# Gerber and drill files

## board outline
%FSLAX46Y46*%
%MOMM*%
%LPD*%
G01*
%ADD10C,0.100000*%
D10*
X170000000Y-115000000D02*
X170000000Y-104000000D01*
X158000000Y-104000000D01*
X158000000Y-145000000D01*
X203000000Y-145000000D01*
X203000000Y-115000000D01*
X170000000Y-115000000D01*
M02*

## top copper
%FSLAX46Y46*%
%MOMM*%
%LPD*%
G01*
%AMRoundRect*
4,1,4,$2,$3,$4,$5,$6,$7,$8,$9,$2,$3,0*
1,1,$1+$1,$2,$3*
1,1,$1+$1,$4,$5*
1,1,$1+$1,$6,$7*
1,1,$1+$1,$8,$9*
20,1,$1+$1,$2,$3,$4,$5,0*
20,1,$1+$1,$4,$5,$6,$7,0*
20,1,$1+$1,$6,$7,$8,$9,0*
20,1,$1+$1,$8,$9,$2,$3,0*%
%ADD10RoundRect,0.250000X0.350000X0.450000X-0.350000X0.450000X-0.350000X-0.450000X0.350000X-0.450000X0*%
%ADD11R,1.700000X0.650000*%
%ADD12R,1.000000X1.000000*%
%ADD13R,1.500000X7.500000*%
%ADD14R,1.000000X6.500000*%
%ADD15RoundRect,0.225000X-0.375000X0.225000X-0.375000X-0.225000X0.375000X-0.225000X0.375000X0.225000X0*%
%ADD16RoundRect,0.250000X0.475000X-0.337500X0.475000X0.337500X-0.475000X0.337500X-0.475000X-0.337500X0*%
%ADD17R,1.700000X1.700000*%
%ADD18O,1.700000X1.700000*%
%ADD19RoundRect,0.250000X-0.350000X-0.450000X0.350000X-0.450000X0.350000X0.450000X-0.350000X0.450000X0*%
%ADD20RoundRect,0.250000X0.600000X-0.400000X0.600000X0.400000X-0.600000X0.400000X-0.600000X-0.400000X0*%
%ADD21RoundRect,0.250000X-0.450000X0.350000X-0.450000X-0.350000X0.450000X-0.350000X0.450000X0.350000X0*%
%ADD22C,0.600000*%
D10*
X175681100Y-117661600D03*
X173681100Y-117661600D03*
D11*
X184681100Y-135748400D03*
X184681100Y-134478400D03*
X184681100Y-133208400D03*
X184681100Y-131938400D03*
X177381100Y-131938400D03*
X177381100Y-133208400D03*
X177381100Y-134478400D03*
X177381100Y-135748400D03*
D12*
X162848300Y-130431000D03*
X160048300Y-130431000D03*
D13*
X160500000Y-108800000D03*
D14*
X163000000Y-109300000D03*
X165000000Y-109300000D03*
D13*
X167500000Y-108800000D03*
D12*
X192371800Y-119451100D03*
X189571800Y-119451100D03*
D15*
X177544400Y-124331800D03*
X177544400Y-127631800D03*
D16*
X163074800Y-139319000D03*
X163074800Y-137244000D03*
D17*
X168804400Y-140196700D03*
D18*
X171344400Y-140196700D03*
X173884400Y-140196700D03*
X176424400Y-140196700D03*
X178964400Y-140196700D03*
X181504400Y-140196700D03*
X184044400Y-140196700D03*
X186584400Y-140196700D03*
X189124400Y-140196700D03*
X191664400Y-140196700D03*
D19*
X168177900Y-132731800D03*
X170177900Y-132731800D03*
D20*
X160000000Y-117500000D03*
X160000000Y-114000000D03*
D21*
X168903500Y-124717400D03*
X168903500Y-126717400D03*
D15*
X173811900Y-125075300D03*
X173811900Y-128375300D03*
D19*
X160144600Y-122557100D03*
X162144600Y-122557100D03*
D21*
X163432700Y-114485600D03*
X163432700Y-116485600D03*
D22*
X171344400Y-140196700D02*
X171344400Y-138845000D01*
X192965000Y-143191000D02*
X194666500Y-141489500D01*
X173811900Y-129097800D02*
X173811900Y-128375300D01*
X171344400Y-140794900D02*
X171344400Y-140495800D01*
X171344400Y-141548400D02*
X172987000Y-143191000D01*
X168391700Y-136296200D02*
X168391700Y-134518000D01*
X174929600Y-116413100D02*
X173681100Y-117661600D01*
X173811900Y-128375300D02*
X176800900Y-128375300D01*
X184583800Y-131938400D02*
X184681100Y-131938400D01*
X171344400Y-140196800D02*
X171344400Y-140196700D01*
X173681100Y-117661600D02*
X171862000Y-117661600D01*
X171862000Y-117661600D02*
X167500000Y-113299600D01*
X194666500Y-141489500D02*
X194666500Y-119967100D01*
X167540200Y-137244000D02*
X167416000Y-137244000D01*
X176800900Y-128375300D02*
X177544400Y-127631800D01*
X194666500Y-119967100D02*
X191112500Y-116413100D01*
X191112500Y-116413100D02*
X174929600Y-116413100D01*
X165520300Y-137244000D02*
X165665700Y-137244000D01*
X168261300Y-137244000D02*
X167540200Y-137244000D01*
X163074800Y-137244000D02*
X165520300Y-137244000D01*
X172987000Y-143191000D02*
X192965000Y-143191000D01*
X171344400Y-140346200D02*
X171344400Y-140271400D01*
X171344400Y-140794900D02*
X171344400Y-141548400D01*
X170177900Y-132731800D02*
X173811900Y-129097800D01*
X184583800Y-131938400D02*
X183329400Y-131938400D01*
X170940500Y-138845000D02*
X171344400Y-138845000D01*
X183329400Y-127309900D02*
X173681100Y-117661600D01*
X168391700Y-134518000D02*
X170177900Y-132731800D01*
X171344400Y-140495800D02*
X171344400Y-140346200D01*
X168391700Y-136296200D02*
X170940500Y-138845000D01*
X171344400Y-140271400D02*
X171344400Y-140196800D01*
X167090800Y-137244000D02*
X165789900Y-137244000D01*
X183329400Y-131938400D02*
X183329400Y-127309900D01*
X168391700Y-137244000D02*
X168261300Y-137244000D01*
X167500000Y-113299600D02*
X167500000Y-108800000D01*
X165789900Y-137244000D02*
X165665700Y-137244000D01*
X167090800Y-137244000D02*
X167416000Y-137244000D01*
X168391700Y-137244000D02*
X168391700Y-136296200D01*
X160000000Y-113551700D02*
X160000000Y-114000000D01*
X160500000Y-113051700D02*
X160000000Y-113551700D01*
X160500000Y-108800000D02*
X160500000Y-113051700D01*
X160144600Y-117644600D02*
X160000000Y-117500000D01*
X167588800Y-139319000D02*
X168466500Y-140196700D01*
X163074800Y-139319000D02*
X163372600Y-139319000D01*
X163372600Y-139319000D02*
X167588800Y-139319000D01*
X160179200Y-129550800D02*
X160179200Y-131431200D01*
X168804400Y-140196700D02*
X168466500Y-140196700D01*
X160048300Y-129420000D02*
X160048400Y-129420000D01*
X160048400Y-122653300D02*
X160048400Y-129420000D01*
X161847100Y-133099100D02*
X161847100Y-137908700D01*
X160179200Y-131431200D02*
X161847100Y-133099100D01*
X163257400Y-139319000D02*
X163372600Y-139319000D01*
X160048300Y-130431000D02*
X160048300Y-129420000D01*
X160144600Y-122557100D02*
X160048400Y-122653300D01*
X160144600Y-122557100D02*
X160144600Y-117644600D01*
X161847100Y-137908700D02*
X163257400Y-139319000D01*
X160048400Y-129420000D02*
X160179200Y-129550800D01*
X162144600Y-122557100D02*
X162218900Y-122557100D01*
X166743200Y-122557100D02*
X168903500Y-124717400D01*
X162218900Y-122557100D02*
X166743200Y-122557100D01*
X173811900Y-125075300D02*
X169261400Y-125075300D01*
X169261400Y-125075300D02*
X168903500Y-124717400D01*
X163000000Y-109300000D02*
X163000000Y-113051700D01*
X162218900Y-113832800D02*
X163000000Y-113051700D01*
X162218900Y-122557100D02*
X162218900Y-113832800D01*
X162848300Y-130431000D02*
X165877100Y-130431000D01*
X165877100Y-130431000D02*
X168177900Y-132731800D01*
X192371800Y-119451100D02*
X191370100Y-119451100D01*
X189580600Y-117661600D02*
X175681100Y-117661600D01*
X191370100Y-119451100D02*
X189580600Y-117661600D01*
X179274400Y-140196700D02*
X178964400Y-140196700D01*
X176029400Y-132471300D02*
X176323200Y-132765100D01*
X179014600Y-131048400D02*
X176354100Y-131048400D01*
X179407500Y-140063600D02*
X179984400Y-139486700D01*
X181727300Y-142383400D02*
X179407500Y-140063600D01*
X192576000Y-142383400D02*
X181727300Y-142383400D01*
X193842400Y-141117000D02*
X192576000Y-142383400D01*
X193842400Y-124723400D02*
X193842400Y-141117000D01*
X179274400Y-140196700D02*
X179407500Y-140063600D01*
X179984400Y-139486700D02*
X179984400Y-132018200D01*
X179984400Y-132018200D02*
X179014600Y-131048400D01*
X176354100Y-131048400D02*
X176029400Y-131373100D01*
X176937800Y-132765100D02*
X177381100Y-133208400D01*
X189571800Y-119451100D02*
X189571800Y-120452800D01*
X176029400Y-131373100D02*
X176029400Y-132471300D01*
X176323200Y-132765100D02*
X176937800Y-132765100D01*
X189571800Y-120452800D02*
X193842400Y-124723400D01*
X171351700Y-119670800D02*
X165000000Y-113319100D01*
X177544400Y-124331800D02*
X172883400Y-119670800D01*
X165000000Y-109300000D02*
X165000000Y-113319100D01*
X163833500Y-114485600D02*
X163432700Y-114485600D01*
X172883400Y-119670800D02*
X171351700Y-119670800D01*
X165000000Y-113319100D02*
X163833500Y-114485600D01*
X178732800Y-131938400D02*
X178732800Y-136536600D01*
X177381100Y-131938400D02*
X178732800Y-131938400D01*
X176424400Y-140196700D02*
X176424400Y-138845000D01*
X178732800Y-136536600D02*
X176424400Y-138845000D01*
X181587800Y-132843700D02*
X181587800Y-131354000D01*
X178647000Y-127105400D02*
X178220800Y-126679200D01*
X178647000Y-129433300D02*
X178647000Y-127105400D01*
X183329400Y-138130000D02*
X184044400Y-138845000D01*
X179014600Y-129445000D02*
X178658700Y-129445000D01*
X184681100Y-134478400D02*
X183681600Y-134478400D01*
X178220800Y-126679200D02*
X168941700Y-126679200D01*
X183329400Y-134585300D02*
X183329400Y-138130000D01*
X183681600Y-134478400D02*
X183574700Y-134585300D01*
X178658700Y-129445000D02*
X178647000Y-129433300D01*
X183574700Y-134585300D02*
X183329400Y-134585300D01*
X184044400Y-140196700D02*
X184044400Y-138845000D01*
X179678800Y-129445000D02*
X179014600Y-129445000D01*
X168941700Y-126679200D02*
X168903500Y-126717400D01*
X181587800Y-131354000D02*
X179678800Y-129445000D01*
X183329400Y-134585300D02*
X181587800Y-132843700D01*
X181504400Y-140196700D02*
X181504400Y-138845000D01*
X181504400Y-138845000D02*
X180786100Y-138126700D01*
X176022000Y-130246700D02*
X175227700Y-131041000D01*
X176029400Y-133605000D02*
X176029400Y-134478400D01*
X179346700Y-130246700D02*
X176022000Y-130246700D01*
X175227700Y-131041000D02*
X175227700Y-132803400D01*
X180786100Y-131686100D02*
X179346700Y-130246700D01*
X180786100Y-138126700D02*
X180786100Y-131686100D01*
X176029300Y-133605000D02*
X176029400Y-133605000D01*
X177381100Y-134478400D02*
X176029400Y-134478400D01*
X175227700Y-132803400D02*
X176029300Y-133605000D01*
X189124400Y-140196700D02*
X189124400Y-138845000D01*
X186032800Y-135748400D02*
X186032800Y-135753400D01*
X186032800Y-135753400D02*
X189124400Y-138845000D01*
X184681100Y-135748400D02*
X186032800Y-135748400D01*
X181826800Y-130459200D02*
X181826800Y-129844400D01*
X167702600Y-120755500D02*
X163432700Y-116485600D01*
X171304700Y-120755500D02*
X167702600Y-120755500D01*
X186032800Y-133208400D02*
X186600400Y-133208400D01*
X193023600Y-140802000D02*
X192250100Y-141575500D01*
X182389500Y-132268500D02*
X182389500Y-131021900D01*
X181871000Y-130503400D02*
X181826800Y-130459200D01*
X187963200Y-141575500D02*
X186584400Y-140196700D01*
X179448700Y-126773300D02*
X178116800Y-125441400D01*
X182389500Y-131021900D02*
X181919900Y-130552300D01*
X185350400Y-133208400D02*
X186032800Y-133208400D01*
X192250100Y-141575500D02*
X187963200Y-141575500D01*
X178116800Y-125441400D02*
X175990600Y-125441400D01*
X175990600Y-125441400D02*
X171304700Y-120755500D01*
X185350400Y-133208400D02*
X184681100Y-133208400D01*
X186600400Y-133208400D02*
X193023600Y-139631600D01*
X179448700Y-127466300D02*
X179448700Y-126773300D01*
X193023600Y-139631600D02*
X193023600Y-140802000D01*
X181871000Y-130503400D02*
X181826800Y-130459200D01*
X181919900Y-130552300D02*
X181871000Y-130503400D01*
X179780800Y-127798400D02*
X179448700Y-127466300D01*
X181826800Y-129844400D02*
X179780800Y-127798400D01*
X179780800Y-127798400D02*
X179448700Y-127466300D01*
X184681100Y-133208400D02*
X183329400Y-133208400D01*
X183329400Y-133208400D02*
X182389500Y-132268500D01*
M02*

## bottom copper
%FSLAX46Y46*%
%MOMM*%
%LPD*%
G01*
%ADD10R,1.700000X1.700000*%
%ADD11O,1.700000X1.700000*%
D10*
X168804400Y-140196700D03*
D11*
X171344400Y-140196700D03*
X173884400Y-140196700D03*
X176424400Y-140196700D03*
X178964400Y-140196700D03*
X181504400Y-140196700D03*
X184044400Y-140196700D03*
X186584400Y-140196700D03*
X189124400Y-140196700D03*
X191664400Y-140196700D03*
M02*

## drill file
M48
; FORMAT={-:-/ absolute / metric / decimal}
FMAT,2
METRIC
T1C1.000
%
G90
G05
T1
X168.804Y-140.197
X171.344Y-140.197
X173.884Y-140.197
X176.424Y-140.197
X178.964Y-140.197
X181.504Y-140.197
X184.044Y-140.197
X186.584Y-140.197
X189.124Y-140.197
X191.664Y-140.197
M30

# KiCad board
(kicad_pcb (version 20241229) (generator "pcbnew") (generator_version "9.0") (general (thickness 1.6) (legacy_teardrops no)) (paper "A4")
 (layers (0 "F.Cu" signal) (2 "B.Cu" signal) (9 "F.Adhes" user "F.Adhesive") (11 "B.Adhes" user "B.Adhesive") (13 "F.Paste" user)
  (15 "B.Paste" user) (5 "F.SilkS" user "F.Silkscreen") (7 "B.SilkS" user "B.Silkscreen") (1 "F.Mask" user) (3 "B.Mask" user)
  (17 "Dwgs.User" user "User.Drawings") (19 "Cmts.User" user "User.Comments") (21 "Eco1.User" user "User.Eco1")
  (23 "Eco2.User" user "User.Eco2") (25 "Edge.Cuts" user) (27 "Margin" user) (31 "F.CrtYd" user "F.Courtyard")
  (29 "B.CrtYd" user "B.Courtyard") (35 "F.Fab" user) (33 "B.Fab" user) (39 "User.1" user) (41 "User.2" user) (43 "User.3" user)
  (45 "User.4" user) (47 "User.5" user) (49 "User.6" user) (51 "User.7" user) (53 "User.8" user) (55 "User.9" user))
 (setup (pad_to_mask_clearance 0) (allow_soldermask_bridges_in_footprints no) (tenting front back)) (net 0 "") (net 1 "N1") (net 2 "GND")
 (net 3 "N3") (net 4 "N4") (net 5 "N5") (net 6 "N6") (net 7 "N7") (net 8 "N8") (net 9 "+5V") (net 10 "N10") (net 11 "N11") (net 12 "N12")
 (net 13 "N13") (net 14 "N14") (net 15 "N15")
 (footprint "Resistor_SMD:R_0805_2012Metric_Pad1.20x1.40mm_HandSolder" (layer "F.Cu") (at 174.6811 117.6616 180)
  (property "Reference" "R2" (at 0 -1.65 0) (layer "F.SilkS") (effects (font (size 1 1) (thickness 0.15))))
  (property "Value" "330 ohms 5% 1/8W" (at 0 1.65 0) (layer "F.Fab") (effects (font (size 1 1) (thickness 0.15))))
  (pad "1" smd roundrect (at -1 0 180) (size 1.2 1.4) (layers "F.Cu" "F.Mask" "F.Paste") (roundrect_rratio 0.208333) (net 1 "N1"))
  (pad "2" smd roundrect (at 1 0 180) (size 1.2 1.4) (layers "F.Cu" "F.Mask" "F.Paste") (roundrect_rratio 0.208333) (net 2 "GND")))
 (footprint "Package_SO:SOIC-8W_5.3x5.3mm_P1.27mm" (layer "F.Cu") (at 181.0311 133.8434 180)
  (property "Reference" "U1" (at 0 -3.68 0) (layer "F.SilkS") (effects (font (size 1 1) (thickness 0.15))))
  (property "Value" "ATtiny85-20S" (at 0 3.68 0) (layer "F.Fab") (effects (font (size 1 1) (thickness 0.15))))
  (pad "1" smd rect (at -3.65 -1.905 180) (size 1.7 0.65) (layers "F.Cu" "F.Mask" "F.Paste") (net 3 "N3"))
  (pad "2" smd rect (at -3.65 -0.635 180) (size 1.7 0.65) (layers "F.Cu" "F.Mask" "F.Paste") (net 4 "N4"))
  (pad "3" smd rect (at -3.65 0.635 180) (size 1.7 0.65) (layers "F.Cu" "F.Mask" "F.Paste") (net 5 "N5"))
  (pad "4" smd rect (at -3.65 1.905 180) (size 1.7 0.65) (layers "F.Cu" "F.Mask" "F.Paste") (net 2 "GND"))
  (pad "5" smd rect (at 3.65 1.905 180) (size 1.7 0.65) (layers "F.Cu" "F.Mask" "F.Paste") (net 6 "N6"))
  (pad "6" smd rect (at 3.65 0.635 180) (size 1.7 0.65) (layers "F.Cu" "F.Mask" "F.Paste") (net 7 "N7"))
  (pad "7" smd rect (at 3.65 -0.635 180) (size 1.7 0.65) (layers "F.Cu" "F.Mask" "F.Paste") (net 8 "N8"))
  (pad "8" smd rect (at 3.65 -1.905 180) (size 1.7 0.65) (layers "F.Cu" "F.Mask" "F.Paste") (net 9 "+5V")))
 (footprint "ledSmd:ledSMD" (layer "F.Cu") (at 161.0483 130.431 180)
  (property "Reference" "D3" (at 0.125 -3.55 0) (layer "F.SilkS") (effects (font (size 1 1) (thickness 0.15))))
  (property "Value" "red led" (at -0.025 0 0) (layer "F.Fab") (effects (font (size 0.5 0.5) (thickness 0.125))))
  (pad "1" smd rect (at -1.8 0 180) (size 1 1) (layers "F.Cu" "F.Mask" "F.Paste") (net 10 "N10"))
  (pad "2" smd rect (at 1 0 180) (size 1 1) (layers "F.Cu" "F.Mask" "F.Paste") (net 9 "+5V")))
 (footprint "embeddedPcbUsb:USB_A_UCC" (layer "F.Cu") (at 164 109 -90)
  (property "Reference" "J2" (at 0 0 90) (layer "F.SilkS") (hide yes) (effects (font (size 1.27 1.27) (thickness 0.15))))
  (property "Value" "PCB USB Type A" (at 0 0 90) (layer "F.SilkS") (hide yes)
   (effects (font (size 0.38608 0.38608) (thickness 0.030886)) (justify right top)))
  (pad "1" smd rect (at -0.2 3.5 270) (size 7.5 1.5) (layers "F.Cu" "F.Mask" "F.Paste") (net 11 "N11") (solder_mask_margin 0.1016))
  (pad "2" smd rect (at 0.3 1 270) (size 6.5 1) (layers "F.Cu" "F.Mask" "F.Paste") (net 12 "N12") (solder_mask_margin 0.1016))
  (pad "3" smd rect (at 0.3 -1 270) (size 6.5 1) (layers "F.Cu" "F.Mask" "F.Paste") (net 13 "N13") (solder_mask_margin 0.1016))
  (pad "4" smd rect (at -0.2 -3.5 270) (size 7.5 1.5) (layers "F.Cu" "F.Mask" "F.Paste") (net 2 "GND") (solder_mask_margin 0.1016)))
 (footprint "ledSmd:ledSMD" (layer "F.Cu") (at 190.5718 119.4511 180)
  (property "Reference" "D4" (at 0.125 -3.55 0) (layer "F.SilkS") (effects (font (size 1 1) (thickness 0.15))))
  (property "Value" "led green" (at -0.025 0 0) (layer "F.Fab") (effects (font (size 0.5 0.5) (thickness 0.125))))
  (pad "1" smd rect (at -1.8 0 180) (size 1 1) (layers "F.Cu" "F.Mask" "F.Paste") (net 1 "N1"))
  (pad "2" smd rect (at 1 0 180) (size 1 1) (layers "F.Cu" "F.Mask" "F.Paste") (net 7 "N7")))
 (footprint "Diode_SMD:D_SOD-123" (layer "F.Cu") (at 177.5444 125.9818 -90)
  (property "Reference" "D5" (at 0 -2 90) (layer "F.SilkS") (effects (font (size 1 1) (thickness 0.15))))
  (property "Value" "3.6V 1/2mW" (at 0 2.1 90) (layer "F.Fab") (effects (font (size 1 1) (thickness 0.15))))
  (pad "1" smd roundrect (at -1.65 0 270) (size 0.9 1.2) (layers "F.Cu" "F.Mask" "F.Paste") (roundrect_rratio 0.25) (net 13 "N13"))
  (pad "2" smd roundrect (at 1.65 0 270) (size 0.9 1.2) (layers "F.Cu" "F.Mask" "F.Paste") (roundrect_rratio 0.25) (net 2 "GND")))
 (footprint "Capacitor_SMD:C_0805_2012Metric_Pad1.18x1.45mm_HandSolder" (layer "F.Cu") (at 163.0748 138.2815 90)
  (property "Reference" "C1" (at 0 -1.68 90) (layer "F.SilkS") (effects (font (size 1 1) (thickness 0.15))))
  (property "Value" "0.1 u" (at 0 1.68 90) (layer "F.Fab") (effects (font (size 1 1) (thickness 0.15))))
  (pad "1" smd roundrect (at -1.0375 0 90) (size 1.175 1.45) (layers "F.Cu" "F.Mask" "F.Paste") (roundrect_rratio 0.212766) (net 9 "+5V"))
  (pad "2" smd roundrect (at 1.0375 0 90) (size 1.175 1.45) (layers "F.Cu" "F.Mask" "F.Paste") (roundrect_rratio 0.212766) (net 2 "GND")))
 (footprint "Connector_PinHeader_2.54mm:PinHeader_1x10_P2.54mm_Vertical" (layer "F.Cu") (at 168.8044 140.1967 90)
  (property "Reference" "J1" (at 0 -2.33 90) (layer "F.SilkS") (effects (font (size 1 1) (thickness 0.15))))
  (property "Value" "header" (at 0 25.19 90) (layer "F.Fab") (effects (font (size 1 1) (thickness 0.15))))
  (pad "1" thru_hole rect (at 0 0 90) (size 1.7 1.7) (drill 1) (layers "*.Cu" "*.Mask") (remove_unused_layers no) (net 9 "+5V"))
  (pad "2" thru_hole oval (at 0 2.54 90) (size 1.7 1.7) (drill 1) (layers "*.Cu" "*.Mask") (remove_unused_layers no) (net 2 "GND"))
  (pad "3" thru_hole oval (at 0 5.08 90) (size 1.7 1.7) (drill 1) (layers "*.Cu" "*.Mask") (remove_unused_layers no) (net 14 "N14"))
  (pad "4" thru_hole oval (at 0 7.62 90) (size 1.7 1.7) (drill 1) (layers "*.Cu" "*.Mask") (remove_unused_layers no) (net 6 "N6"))
  (pad "5" thru_hole oval (at 0 10.16 90) (size 1.7 1.7) (drill 1) (layers "*.Cu" "*.Mask") (remove_unused_layers no) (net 7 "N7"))
  (pad "6" thru_hole oval (at 0 12.7 90) (size 1.7 1.7) (drill 1) (layers "*.Cu" "*.Mask") (remove_unused_layers no) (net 8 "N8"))
  (pad "7" thru_hole oval (at 0 15.24 90) (size 1.7 1.7) (drill 1) (layers "*.Cu" "*.Mask") (remove_unused_layers no) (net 4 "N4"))
  (pad "8" thru_hole oval (at 0 17.78 90) (size 1.7 1.7) (drill 1) (layers "*.Cu" "*.Mask") (remove_unused_layers no) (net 5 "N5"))
  (pad "9" thru_hole oval (at 0 20.32 90) (size 1.7 1.7) (drill 1) (layers "*.Cu" "*.Mask") (remove_unused_layers no) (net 3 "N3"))
  (pad "10" thru_hole oval (at 0 22.86 90) (size 1.7 1.7) (drill 1) (layers "*.Cu" "*.Mask") (remove_unused_layers no) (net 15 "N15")))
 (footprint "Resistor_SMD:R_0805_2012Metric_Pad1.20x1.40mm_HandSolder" (layer "F.Cu") (at 169.1779 132.7318)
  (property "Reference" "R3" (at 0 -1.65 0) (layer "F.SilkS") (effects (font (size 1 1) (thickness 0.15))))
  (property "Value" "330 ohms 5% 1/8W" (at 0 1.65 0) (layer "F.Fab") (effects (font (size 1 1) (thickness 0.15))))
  (pad "1" smd roundrect (at -1 0) (size 1.2 1.4) (layers "F.Cu" "F.Mask" "F.Paste") (roundrect_rratio 0.208333) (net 10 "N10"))
  (pad "2" smd roundrect (at 1 0) (size 1.2 1.4) (layers "F.Cu" "F.Mask" "F.Paste") (roundrect_rratio 0.208333) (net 2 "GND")))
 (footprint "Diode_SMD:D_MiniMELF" (layer "F.Cu") (at 160 115.75 90)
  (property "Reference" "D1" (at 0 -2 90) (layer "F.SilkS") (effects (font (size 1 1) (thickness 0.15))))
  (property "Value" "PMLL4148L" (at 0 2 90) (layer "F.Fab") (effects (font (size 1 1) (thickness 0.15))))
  (pad "1" smd roundrect (at -1.75 0 90) (size 1.3 1.7) (layers "F.Cu" "F.Mask" "F.Paste") (roundrect_rratio 0.1923076923) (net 9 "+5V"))
  (pad "2" smd roundrect (at 1.75 0 90) (size 1.3 1.7) (layers "F.Cu" "F.Mask" "F.Paste") (roundrect_rratio 0.1923076923) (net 11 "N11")))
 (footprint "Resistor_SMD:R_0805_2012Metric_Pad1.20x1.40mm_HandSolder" (layer "F.Cu") (at 168.9035 125.7174 -90)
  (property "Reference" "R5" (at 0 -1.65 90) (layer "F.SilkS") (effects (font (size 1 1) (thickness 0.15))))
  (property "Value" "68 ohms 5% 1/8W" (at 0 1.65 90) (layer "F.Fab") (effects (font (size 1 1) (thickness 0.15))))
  (pad "1" smd roundrect (at -1 0 270) (size 1.2 1.4) (layers "F.Cu" "F.Mask" "F.Paste") (roundrect_rratio 0.208333) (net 12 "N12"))
  (pad "2" smd roundrect (at 1 0 270) (size 1.2 1.4) (layers "F.Cu" "F.Mask" "F.Paste") (roundrect_rratio 0.208333) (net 4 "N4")))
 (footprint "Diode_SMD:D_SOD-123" (layer "F.Cu") (at 173.8119 126.7253 -90)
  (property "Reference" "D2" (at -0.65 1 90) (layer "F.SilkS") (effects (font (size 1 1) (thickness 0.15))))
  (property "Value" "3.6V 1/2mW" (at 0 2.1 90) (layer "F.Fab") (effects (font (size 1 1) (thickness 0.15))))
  (pad "1" smd roundrect (at -1.65 0 270) (size 0.9 1.2) (layers "F.Cu" "F.Mask" "F.Paste") (roundrect_rratio 0.25) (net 12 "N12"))
  (pad "2" smd roundrect (at 1.65 0 270) (size 0.9 1.2) (layers "F.Cu" "F.Mask" "F.Paste") (roundrect_rratio 0.25) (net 2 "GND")))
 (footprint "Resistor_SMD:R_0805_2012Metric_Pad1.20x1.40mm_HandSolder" (layer "F.Cu") (at 161.1446 122.5571)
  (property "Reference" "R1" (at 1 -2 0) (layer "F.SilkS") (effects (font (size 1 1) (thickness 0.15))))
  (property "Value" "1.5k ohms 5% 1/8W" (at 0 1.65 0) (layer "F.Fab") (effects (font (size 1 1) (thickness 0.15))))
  (pad "1" smd roundrect (at -1 0) (size 1.2 1.4) (layers "F.Cu" "F.Mask" "F.Paste") (roundrect_rratio 0.208333) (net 9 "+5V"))
  (pad "2" smd roundrect (at 1 0) (size 1.2 1.4) (layers "F.Cu" "F.Mask" "F.Paste") (roundrect_rratio 0.208333) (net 12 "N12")))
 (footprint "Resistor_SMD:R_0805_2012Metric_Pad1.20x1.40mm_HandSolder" (layer "F.Cu") (at 163.4327 115.4856 -90)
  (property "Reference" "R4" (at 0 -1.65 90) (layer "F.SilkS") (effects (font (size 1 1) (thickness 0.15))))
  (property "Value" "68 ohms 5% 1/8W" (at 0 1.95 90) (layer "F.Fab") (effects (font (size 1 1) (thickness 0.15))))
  (pad "1" smd roundrect (at -1 0 270) (size 1.2 1.4) (layers "F.Cu" "F.Mask" "F.Paste") (roundrect_rratio 0.208333) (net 13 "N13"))
  (pad "2" smd roundrect (at 1 0 270) (size 1.2 1.4) (layers "F.Cu" "F.Mask" "F.Paste") (roundrect_rratio 0.208333) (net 5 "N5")))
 (gr_poly
  (pts (xy 170 115) (xy 170 104) (xy 158 104) (xy 158 145) (xy 203 145) (xy 203 115)) (stroke (width 0.1) (type solid)) (fill no)
  (layer "Edge.Cuts"))
 (segment (start 171.3444 140.1967) (end 171.3444 138.845) (width 0.6) (layer "F.Cu") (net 2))
 (segment (start 192.965 143.191) (end 194.6665 141.4895) (width 0.6) (layer "F.Cu") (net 2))
 (segment (start 173.8119 129.0978) (end 173.8119 128.3753) (width 0.6) (layer "F.Cu") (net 2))
 (segment (start 171.3444 140.7949) (end 171.3444 140.4958) (width 0.6) (layer "F.Cu") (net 2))
 (segment (start 171.3444 141.5484) (end 172.987 143.191) (width 0.6) (layer "F.Cu") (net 2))
 (segment (start 168.3917 136.2962) (end 168.3917 134.518) (width 0.6) (layer "F.Cu") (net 2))
 (segment (start 174.9296 116.4131) (end 173.6811 117.6616) (width 0.6) (layer "F.Cu") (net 2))
 (segment (start 173.8119 128.3753) (end 176.8009 128.3753) (width 0.6) (layer "F.Cu") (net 2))
 (segment (start 184.5838 131.9384) (end 184.6811 131.9384) (width 0.6) (layer "F.Cu") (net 2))
 (segment (start 171.3444 140.1968) (end 171.3444 140.1967) (width 0.6) (layer "F.Cu") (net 2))
 (segment (start 173.6811 117.6616) (end 171.862 117.6616) (width 0.6) (layer "F.Cu") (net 2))
 (segment (start 171.862 117.6616) (end 167.5 113.2996) (width 0.6) (layer "F.Cu") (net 2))
 (segment (start 194.6665 141.4895) (end 194.6665 119.9671) (width 0.6) (layer "F.Cu") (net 2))
 (segment (start 167.5402 137.244) (end 167.416 137.244) (width 0.6) (layer "F.Cu") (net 2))
 (segment (start 176.8009 128.3753) (end 177.5444 127.6318) (width 0.6) (layer "F.Cu") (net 2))
 (segment (start 194.6665 119.9671) (end 191.1125 116.4131) (width 0.6) (layer "F.Cu") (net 2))
 (segment (start 191.1125 116.4131) (end 174.9296 116.4131) (width 0.6) (layer "F.Cu") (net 2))
 (segment (start 165.5203 137.244) (end 165.6657 137.244) (width 0.6) (layer "F.Cu") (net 2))
 (segment (start 168.2613 137.244) (end 167.5402 137.244) (width 0.6) (layer "F.Cu") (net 2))
 (segment (start 163.0748 137.244) (end 165.5203 137.244) (width 0.6) (layer "F.Cu") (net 2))
 (segment (start 172.987 143.191) (end 192.965 143.191) (width 0.6) (layer "F.Cu") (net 2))
 (segment (start 171.3444 140.3462) (end 171.3444 140.2714) (width 0.6) (layer "F.Cu") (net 2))
 (segment (start 171.3444 140.7949) (end 171.3444 141.5484) (width 0.6) (layer "F.Cu") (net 2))
 (segment (start 170.1779 132.7318) (end 173.8119 129.0978) (width 0.6) (layer "F.Cu") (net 2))
 (segment (start 184.5838 131.9384) (end 183.3294 131.9384) (width 0.6) (layer "F.Cu") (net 2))
 (segment (start 170.9405 138.845) (end 171.3444 138.845) (width 0.6) (layer "F.Cu") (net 2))
 (segment (start 183.3294 127.3099) (end 173.6811 117.6616) (width 0.6) (layer "F.Cu") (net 2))
 (segment (start 168.3917 134.518) (end 170.1779 132.7318) (width 0.6) (layer "F.Cu") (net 2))
 (segment (start 171.3444 140.4958) (end 171.3444 140.3462) (width 0.6) (layer "F.Cu") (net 2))
 (segment (start 168.3917 136.2962) (end 170.9405 138.845) (width 0.6) (layer "F.Cu") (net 2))
 (segment (start 171.3444 140.2714) (end 171.3444 140.1968) (width 0.6) (layer "F.Cu") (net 2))
 (segment (start 167.0908 137.244) (end 165.7899 137.244) (width 0.6) (layer "F.Cu") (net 2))
 (segment (start 183.3294 131.9384) (end 183.3294 127.3099) (width 0.6) (layer "F.Cu") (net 2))
 (segment (start 168.3917 137.244) (end 168.2613 137.244) (width 0.6) (layer "F.Cu") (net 2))
 (segment (start 167.5 113.2996) (end 167.5 108.8) (width 0.6) (layer "F.Cu") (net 2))
 (segment (start 165.7899 137.244) (end 165.6657 137.244) (width 0.6) (layer "F.Cu") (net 2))
 (segment (start 167.0908 137.244) (end 167.416 137.244) (width 0.6) (layer "F.Cu") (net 2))
 (segment (start 168.3917 137.244) (end 168.3917 136.2962) (width 0.6) (layer "F.Cu") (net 2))
 (segment (start 160 113.5517) (end 160 114) (width 0.6) (layer "F.Cu") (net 11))
 (segment (start 160.5 113.0517) (end 160 113.5517) (width 0.6) (layer "F.Cu") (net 11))
 (segment (start 160.5 108.8) (end 160.5 113.0517) (width 0.6) (layer "F.Cu") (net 11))
 (segment (start 160.1446 117.6446) (end 160 117.5) (width 0.6) (layer "F.Cu") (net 9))
 (segment (start 167.5888 139.319) (end 168.4665 140.1967) (width 0.6) (layer "F.Cu") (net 9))
 (segment (start 163.0748 139.319) (end 163.3726 139.319) (width 0.6) (layer "F.Cu") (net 9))
 (segment (start 163.3726 139.319) (end 167.5888 139.319) (width 0.6) (layer "F.Cu") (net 9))
 (segment (start 160.1792 129.5508) (end 160.1792 131.4312) (width 0.6) (layer "F.Cu") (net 9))
 (segment (start 168.8044 140.1967) (end 168.4665 140.1967) (width 0.6) (layer "F.Cu") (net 9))
 (segment (start 160.0483 129.42) (end 160.0484 129.42) (width 0.6) (layer "F.Cu") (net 9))
 (segment (start 160.0484 122.6533) (end 160.0484 129.42) (width 0.6) (layer "F.Cu") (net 9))
 (segment (start 161.8471 133.0991) (end 161.8471 137.9087) (width 0.6) (layer "F.Cu") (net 9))
 (segment (start 160.1792 131.4312) (end 161.8471 133.0991) (width 0.6) (layer "F.Cu") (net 9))
 (segment (start 163.2574 139.319) (end 163.3726 139.319) (width 0.6) (layer "F.Cu") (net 9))
 (segment (start 160.0483 130.431) (end 160.0483 129.42) (width 0.6) (layer "F.Cu") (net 9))
 (segment (start 160.1446 122.5571) (end 160.0484 122.6533) (width 0.6) (layer "F.Cu") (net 9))
 (segment (start 160.1446 122.5571) (end 160.1446 117.6446) (width 0.6) (layer "F.Cu") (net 9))
 (segment (start 161.8471 137.9087) (end 163.2574 139.319) (width 0.6) (layer "F.Cu") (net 9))
 (segment (start 160.0484 129.42) (end 160.1792 129.5508) (width 0.6) (layer "F.Cu") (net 9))
 (segment (start 162.1446 122.5571) (end 162.2189 122.5571) (width 0.6) (layer "F.Cu") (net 12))
 (segment (start 166.7432 122.5571) (end 168.9035 124.7174) (width 0.6) (layer "F.Cu") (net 12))
 (segment (start 162.2189 122.5571) (end 166.7432 122.5571) (width 0.6) (layer "F.Cu") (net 12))
 (segment (start 173.8119 125.0753) (end 169.2614 125.0753) (width 0.6) (layer "F.Cu") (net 12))
 (segment (start 169.2614 125.0753) (end 168.9035 124.7174) (width 0.6) (layer "F.Cu") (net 12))
 (segment (start 163 109.3) (end 163 113.0517) (width 0.6) (layer "F.Cu") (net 12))
 (segment (start 162.2189 113.8328) (end 163 113.0517) (width 0.6) (layer "F.Cu") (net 12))
 (segment (start 162.2189 122.5571) (end 162.2189 113.8328) (width 0.6) (layer "F.Cu") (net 12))
 (segment (start 162.8483 130.431) (end 165.8771 130.431) (width 0.6) (layer "F.Cu") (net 10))
 (segment (start 165.8771 130.431) (end 168.1779 132.7318) (width 0.6) (layer "F.Cu") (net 10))
 (segment (start 192.3718 119.4511) (end 191.3701 119.4511) (width 0.6) (layer "F.Cu") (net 1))
 (segment (start 189.5806 117.6616) (end 175.6811 117.6616) (width 0.6) (layer "F.Cu") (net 1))
 (segment (start 191.3701 119.4511) (end 189.5806 117.6616) (width 0.6) (layer "F.Cu") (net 1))
 (segment (start 179.2744 140.1967) (end 178.9644 140.1967) (width 0.6) (layer "F.Cu") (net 7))
 (segment (start 176.0294 132.4713) (end 176.3232 132.7651) (width 0.6) (layer "F.Cu") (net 7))
 (segment (start 179.0146 131.0484) (end 176.3541 131.0484) (width 0.6) (layer "F.Cu") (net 7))
 (segment (start 179.4075 140.0636) (end 179.9844 139.4867) (width 0.6) (layer "F.Cu") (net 7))
 (segment (start 181.7273 142.3834) (end 179.4075 140.0636) (width 0.6) (layer "F.Cu") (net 7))
 (segment (start 192.576 142.3834) (end 181.7273 142.3834) (width 0.6) (layer "F.Cu") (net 7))
 (segment (start 193.8424 141.117) (end 192.576 142.3834) (width 0.6) (layer "F.Cu") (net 7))
 (segment (start 193.8424 124.7234) (end 193.8424 141.117) (width 0.6) (layer "F.Cu") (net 7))
 (segment (start 179.2744 140.1967) (end 179.4075 140.0636) (width 0.6) (layer "F.Cu") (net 7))
 (segment (start 179.9844 139.4867) (end 179.9844 132.0182) (width 0.6) (layer "F.Cu") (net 7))
 (segment (start 179.9844 132.0182) (end 179.0146 131.0484) (width 0.6) (layer "F.Cu") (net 7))
 (segment (start 176.3541 131.0484) (end 176.0294 131.3731) (width 0.6) (layer "F.Cu") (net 7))
 (segment (start 176.9378 132.7651) (end 177.3811 133.2084) (width 0.6) (layer "F.Cu") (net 7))
 (segment (start 189.5718 119.4511) (end 189.5718 120.4528) (width 0.6) (layer "F.Cu") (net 7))
 (segment (start 176.0294 131.3731) (end 176.0294 132.4713) (width 0.6) (layer "F.Cu") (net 7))
 (segment (start 176.3232 132.7651) (end 176.9378 132.7651) (width 0.6) (layer "F.Cu") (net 7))
 (segment (start 189.5718 120.4528) (end 193.8424 124.7234) (width 0.6) (layer "F.Cu") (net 7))
 (segment (start 171.3517 119.6708) (end 165 113.3191) (width 0.6) (layer "F.Cu") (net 13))
 (segment (start 177.5444 124.3318) (end 172.8834 119.6708) (width 0.6) (layer "F.Cu") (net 13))
 (segment (start 165 109.3) (end 165 113.3191) (width 0.6) (layer "F.Cu") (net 13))
 (segment (start 163.8335 114.4856) (end 163.4327 114.4856) (width 0.6) (layer "F.Cu") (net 13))
 (segment (start 172.8834 119.6708) (end 171.3517 119.6708) (width 0.6) (layer "F.Cu") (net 13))
 (segment (start 165 113.3191) (end 163.8335 114.4856) (width 0.6) (layer "F.Cu") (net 13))
 (segment (start 178.7328 131.9384) (end 178.7328 136.5366) (width 0.6) (layer "F.Cu") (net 6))
 (segment (start 177.3811 131.9384) (end 178.7328 131.9384) (width 0.6) (layer "F.Cu") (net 6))
 (segment (start 176.4244 140.1967) (end 176.4244 138.845) (width 0.6) (layer "F.Cu") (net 6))
 (segment (start 178.7328 136.5366) (end 176.4244 138.845) (width 0.6) (layer "F.Cu") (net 6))
 (segment (start 181.5878 132.8437) (end 181.5878 131.354) (width 0.6) (layer "F.Cu") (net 4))
 (segment (start 178.647 127.1054) (end 178.2208 126.6792) (width 0.6) (layer "F.Cu") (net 4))
 (segment (start 178.647 129.4333) (end 178.647 127.1054) (width 0.6) (layer "F.Cu") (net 4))
 (segment (start 183.3294 138.13) (end 184.0444 138.845) (width 0.6) (layer "F.Cu") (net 4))
 (segment (start 179.0146 129.445) (end 178.6587 129.445) (width 0.6) (layer "F.Cu") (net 4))
 (segment (start 184.6811 134.4784) (end 183.6816 134.4784) (width 0.6) (layer "F.Cu") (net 4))
 (segment (start 178.2208 126.6792) (end 168.9417 126.6792) (width 0.6) (layer "F.Cu") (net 4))
 (segment (start 183.3294 134.5853) (end 183.3294 138.13) (width 0.6) (layer "F.Cu") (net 4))
 (segment (start 183.6816 134.4784) (end 183.5747 134.5853) (width 0.6) (layer "F.Cu") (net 4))
 (segment (start 178.6587 129.445) (end 178.647 129.4333) (width 0.6) (layer "F.Cu") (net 4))
 (segment (start 183.5747 134.5853) (end 183.3294 134.5853) (width 0.6) (layer "F.Cu") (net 4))
 (segment (start 184.0444 140.1967) (end 184.0444 138.845) (width 0.6) (layer "F.Cu") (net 4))
 (segment (start 179.6788 129.445) (end 179.0146 129.445) (width 0.6) (layer "F.Cu") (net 4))
 (segment (start 168.9417 126.6792) (end 168.9035 126.7174) (width 0.6) (layer "F.Cu") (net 4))
 (segment (start 181.5878 131.354) (end 179.6788 129.445) (width 0.6) (layer "F.Cu") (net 4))
 (segment (start 183.3294 134.5853) (end 181.5878 132.8437) (width 0.6) (layer "F.Cu") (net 4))
 (segment (start 181.5044 140.1967) (end 181.5044 138.845) (width 0.6) (layer "F.Cu") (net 8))
 (segment (start 181.5044 138.845) (end 180.7861 138.1267) (width 0.6) (layer "F.Cu") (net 8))
 (segment (start 176.022 130.2467) (end 175.2277 131.041) (width 0.6) (layer "F.Cu") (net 8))
 (segment (start 176.0294 133.605) (end 176.0294 134.4784) (width 0.6) (layer "F.Cu") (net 8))
 (segment (start 179.3467 130.2467) (end 176.022 130.2467) (width 0.6) (layer "F.Cu") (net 8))
 (segment (start 175.2277 131.041) (end 175.2277 132.8034) (width 0.6) (layer "F.Cu") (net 8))
 (segment (start 180.7861 131.6861) (end 179.3467 130.2467) (width 0.6) (layer "F.Cu") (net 8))
 (segment (start 180.7861 138.1267) (end 180.7861 131.6861) (width 0.6) (layer "F.Cu") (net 8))
 (segment (start 176.0293 133.605) (end 176.0294 133.605) (width 0.6) (layer "F.Cu") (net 8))
 (segment (start 177.3811 134.4784) (end 176.0294 134.4784) (width 0.6) (layer "F.Cu") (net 8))
 (segment (start 175.2277 132.8034) (end 176.0293 133.605) (width 0.6) (layer "F.Cu") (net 8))
 (segment (start 189.1244 140.1967) (end 189.1244 138.845) (width 0.6) (layer "F.Cu") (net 3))
 (segment (start 186.0328 135.7484) (end 186.0328 135.7534) (width 0.6) (layer "F.Cu") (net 3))
 (segment (start 186.0328 135.7534) (end 189.1244 138.845) (width 0.6) (layer "F.Cu") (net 3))
 (segment (start 184.6811 135.7484) (end 186.0328 135.7484) (width 0.6) (layer "F.Cu") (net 3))
 (segment (start 181.8268 130.4592) (end 181.8268 129.8444) (width 0.6) (layer "F.Cu") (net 5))
 (segment (start 167.7026 120.7555) (end 163.4327 116.4856) (width 0.6) (layer "F.Cu") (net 5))
 (segment (start 171.3047 120.7555) (end 167.7026 120.7555) (width 0.6) (layer "F.Cu") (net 5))
 (segment (start 186.0328 133.2084) (end 186.6004 133.2084) (width 0.6) (layer "F.Cu") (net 5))
 (segment (start 193.0236 140.802) (end 192.2501 141.5755) (width 0.6) (layer "F.Cu") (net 5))
 (segment (start 182.3895 132.2685) (end 182.3895 131.0219) (width 0.6) (layer "F.Cu") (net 5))
 (segment (start 181.871 130.5034) (end 181.8268 130.4592) (width 0.6) (layer "F.Cu") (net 5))
 (segment (start 187.9632 141.5755) (end 186.5844 140.1967) (width 0.6) (layer "F.Cu") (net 5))
 (segment (start 179.4487 126.7733) (end 178.1168 125.4414) (width 0.6) (layer "F.Cu") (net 5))
 (segment (start 182.3895 131.0219) (end 181.9199 130.5523) (width 0.6) (layer "F.Cu") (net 5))
 (segment (start 185.3504 133.2084) (end 186.0328 133.2084) (width 0.6) (layer "F.Cu") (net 5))
 (segment (start 192.2501 141.5755) (end 187.9632 141.5755) (width 0.6) (layer "F.Cu") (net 5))
 (segment (start 178.1168 125.4414) (end 175.9906 125.4414) (width 0.6) (layer "F.Cu") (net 5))
 (segment (start 175.9906 125.4414) (end 171.3047 120.7555) (width 0.6) (layer "F.Cu") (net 5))
 (segment (start 185.3504 133.2084) (end 184.6811 133.2084) (width 0.6) (layer "F.Cu") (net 5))
 (segment (start 186.6004 133.2084) (end 193.0236 139.6316) (width 0.6) (layer "F.Cu") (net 5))
 (segment (start 179.4487 127.4663) (end 179.4487 126.7733) (width 0.6) (layer "F.Cu") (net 5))
 (segment (start 193.0236 139.6316) (end 193.0236 140.802) (width 0.6) (layer "F.Cu") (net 5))
 (segment (start 181.871 130.5034) (end 181.8268 130.4592) (width 0.6) (layer "F.Cu") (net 5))
 (segment (start 181.9199 130.5523) (end 181.871 130.5034) (width 0.6) (layer "F.Cu") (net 5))
 (segment (start 179.7808 127.7984) (end 179.4487 127.4663) (width 0.6) (layer "F.Cu") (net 5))
 (segment (start 181.8268 129.8444) (end 179.7808 127.7984) (width 0.6) (layer "F.Cu") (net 5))
 (segment (start 179.7808 127.7984) (end 179.4487 127.4663) (width 0.6) (layer "F.Cu") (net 5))
 (segment (start 184.6811 133.2084) (end 183.3294 133.2084) (width 0.6) (layer "F.Cu") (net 5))
 (segment (start 183.3294 133.2084) (end 182.3895 132.2685) (width 0.6) (layer "F.Cu") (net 5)))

